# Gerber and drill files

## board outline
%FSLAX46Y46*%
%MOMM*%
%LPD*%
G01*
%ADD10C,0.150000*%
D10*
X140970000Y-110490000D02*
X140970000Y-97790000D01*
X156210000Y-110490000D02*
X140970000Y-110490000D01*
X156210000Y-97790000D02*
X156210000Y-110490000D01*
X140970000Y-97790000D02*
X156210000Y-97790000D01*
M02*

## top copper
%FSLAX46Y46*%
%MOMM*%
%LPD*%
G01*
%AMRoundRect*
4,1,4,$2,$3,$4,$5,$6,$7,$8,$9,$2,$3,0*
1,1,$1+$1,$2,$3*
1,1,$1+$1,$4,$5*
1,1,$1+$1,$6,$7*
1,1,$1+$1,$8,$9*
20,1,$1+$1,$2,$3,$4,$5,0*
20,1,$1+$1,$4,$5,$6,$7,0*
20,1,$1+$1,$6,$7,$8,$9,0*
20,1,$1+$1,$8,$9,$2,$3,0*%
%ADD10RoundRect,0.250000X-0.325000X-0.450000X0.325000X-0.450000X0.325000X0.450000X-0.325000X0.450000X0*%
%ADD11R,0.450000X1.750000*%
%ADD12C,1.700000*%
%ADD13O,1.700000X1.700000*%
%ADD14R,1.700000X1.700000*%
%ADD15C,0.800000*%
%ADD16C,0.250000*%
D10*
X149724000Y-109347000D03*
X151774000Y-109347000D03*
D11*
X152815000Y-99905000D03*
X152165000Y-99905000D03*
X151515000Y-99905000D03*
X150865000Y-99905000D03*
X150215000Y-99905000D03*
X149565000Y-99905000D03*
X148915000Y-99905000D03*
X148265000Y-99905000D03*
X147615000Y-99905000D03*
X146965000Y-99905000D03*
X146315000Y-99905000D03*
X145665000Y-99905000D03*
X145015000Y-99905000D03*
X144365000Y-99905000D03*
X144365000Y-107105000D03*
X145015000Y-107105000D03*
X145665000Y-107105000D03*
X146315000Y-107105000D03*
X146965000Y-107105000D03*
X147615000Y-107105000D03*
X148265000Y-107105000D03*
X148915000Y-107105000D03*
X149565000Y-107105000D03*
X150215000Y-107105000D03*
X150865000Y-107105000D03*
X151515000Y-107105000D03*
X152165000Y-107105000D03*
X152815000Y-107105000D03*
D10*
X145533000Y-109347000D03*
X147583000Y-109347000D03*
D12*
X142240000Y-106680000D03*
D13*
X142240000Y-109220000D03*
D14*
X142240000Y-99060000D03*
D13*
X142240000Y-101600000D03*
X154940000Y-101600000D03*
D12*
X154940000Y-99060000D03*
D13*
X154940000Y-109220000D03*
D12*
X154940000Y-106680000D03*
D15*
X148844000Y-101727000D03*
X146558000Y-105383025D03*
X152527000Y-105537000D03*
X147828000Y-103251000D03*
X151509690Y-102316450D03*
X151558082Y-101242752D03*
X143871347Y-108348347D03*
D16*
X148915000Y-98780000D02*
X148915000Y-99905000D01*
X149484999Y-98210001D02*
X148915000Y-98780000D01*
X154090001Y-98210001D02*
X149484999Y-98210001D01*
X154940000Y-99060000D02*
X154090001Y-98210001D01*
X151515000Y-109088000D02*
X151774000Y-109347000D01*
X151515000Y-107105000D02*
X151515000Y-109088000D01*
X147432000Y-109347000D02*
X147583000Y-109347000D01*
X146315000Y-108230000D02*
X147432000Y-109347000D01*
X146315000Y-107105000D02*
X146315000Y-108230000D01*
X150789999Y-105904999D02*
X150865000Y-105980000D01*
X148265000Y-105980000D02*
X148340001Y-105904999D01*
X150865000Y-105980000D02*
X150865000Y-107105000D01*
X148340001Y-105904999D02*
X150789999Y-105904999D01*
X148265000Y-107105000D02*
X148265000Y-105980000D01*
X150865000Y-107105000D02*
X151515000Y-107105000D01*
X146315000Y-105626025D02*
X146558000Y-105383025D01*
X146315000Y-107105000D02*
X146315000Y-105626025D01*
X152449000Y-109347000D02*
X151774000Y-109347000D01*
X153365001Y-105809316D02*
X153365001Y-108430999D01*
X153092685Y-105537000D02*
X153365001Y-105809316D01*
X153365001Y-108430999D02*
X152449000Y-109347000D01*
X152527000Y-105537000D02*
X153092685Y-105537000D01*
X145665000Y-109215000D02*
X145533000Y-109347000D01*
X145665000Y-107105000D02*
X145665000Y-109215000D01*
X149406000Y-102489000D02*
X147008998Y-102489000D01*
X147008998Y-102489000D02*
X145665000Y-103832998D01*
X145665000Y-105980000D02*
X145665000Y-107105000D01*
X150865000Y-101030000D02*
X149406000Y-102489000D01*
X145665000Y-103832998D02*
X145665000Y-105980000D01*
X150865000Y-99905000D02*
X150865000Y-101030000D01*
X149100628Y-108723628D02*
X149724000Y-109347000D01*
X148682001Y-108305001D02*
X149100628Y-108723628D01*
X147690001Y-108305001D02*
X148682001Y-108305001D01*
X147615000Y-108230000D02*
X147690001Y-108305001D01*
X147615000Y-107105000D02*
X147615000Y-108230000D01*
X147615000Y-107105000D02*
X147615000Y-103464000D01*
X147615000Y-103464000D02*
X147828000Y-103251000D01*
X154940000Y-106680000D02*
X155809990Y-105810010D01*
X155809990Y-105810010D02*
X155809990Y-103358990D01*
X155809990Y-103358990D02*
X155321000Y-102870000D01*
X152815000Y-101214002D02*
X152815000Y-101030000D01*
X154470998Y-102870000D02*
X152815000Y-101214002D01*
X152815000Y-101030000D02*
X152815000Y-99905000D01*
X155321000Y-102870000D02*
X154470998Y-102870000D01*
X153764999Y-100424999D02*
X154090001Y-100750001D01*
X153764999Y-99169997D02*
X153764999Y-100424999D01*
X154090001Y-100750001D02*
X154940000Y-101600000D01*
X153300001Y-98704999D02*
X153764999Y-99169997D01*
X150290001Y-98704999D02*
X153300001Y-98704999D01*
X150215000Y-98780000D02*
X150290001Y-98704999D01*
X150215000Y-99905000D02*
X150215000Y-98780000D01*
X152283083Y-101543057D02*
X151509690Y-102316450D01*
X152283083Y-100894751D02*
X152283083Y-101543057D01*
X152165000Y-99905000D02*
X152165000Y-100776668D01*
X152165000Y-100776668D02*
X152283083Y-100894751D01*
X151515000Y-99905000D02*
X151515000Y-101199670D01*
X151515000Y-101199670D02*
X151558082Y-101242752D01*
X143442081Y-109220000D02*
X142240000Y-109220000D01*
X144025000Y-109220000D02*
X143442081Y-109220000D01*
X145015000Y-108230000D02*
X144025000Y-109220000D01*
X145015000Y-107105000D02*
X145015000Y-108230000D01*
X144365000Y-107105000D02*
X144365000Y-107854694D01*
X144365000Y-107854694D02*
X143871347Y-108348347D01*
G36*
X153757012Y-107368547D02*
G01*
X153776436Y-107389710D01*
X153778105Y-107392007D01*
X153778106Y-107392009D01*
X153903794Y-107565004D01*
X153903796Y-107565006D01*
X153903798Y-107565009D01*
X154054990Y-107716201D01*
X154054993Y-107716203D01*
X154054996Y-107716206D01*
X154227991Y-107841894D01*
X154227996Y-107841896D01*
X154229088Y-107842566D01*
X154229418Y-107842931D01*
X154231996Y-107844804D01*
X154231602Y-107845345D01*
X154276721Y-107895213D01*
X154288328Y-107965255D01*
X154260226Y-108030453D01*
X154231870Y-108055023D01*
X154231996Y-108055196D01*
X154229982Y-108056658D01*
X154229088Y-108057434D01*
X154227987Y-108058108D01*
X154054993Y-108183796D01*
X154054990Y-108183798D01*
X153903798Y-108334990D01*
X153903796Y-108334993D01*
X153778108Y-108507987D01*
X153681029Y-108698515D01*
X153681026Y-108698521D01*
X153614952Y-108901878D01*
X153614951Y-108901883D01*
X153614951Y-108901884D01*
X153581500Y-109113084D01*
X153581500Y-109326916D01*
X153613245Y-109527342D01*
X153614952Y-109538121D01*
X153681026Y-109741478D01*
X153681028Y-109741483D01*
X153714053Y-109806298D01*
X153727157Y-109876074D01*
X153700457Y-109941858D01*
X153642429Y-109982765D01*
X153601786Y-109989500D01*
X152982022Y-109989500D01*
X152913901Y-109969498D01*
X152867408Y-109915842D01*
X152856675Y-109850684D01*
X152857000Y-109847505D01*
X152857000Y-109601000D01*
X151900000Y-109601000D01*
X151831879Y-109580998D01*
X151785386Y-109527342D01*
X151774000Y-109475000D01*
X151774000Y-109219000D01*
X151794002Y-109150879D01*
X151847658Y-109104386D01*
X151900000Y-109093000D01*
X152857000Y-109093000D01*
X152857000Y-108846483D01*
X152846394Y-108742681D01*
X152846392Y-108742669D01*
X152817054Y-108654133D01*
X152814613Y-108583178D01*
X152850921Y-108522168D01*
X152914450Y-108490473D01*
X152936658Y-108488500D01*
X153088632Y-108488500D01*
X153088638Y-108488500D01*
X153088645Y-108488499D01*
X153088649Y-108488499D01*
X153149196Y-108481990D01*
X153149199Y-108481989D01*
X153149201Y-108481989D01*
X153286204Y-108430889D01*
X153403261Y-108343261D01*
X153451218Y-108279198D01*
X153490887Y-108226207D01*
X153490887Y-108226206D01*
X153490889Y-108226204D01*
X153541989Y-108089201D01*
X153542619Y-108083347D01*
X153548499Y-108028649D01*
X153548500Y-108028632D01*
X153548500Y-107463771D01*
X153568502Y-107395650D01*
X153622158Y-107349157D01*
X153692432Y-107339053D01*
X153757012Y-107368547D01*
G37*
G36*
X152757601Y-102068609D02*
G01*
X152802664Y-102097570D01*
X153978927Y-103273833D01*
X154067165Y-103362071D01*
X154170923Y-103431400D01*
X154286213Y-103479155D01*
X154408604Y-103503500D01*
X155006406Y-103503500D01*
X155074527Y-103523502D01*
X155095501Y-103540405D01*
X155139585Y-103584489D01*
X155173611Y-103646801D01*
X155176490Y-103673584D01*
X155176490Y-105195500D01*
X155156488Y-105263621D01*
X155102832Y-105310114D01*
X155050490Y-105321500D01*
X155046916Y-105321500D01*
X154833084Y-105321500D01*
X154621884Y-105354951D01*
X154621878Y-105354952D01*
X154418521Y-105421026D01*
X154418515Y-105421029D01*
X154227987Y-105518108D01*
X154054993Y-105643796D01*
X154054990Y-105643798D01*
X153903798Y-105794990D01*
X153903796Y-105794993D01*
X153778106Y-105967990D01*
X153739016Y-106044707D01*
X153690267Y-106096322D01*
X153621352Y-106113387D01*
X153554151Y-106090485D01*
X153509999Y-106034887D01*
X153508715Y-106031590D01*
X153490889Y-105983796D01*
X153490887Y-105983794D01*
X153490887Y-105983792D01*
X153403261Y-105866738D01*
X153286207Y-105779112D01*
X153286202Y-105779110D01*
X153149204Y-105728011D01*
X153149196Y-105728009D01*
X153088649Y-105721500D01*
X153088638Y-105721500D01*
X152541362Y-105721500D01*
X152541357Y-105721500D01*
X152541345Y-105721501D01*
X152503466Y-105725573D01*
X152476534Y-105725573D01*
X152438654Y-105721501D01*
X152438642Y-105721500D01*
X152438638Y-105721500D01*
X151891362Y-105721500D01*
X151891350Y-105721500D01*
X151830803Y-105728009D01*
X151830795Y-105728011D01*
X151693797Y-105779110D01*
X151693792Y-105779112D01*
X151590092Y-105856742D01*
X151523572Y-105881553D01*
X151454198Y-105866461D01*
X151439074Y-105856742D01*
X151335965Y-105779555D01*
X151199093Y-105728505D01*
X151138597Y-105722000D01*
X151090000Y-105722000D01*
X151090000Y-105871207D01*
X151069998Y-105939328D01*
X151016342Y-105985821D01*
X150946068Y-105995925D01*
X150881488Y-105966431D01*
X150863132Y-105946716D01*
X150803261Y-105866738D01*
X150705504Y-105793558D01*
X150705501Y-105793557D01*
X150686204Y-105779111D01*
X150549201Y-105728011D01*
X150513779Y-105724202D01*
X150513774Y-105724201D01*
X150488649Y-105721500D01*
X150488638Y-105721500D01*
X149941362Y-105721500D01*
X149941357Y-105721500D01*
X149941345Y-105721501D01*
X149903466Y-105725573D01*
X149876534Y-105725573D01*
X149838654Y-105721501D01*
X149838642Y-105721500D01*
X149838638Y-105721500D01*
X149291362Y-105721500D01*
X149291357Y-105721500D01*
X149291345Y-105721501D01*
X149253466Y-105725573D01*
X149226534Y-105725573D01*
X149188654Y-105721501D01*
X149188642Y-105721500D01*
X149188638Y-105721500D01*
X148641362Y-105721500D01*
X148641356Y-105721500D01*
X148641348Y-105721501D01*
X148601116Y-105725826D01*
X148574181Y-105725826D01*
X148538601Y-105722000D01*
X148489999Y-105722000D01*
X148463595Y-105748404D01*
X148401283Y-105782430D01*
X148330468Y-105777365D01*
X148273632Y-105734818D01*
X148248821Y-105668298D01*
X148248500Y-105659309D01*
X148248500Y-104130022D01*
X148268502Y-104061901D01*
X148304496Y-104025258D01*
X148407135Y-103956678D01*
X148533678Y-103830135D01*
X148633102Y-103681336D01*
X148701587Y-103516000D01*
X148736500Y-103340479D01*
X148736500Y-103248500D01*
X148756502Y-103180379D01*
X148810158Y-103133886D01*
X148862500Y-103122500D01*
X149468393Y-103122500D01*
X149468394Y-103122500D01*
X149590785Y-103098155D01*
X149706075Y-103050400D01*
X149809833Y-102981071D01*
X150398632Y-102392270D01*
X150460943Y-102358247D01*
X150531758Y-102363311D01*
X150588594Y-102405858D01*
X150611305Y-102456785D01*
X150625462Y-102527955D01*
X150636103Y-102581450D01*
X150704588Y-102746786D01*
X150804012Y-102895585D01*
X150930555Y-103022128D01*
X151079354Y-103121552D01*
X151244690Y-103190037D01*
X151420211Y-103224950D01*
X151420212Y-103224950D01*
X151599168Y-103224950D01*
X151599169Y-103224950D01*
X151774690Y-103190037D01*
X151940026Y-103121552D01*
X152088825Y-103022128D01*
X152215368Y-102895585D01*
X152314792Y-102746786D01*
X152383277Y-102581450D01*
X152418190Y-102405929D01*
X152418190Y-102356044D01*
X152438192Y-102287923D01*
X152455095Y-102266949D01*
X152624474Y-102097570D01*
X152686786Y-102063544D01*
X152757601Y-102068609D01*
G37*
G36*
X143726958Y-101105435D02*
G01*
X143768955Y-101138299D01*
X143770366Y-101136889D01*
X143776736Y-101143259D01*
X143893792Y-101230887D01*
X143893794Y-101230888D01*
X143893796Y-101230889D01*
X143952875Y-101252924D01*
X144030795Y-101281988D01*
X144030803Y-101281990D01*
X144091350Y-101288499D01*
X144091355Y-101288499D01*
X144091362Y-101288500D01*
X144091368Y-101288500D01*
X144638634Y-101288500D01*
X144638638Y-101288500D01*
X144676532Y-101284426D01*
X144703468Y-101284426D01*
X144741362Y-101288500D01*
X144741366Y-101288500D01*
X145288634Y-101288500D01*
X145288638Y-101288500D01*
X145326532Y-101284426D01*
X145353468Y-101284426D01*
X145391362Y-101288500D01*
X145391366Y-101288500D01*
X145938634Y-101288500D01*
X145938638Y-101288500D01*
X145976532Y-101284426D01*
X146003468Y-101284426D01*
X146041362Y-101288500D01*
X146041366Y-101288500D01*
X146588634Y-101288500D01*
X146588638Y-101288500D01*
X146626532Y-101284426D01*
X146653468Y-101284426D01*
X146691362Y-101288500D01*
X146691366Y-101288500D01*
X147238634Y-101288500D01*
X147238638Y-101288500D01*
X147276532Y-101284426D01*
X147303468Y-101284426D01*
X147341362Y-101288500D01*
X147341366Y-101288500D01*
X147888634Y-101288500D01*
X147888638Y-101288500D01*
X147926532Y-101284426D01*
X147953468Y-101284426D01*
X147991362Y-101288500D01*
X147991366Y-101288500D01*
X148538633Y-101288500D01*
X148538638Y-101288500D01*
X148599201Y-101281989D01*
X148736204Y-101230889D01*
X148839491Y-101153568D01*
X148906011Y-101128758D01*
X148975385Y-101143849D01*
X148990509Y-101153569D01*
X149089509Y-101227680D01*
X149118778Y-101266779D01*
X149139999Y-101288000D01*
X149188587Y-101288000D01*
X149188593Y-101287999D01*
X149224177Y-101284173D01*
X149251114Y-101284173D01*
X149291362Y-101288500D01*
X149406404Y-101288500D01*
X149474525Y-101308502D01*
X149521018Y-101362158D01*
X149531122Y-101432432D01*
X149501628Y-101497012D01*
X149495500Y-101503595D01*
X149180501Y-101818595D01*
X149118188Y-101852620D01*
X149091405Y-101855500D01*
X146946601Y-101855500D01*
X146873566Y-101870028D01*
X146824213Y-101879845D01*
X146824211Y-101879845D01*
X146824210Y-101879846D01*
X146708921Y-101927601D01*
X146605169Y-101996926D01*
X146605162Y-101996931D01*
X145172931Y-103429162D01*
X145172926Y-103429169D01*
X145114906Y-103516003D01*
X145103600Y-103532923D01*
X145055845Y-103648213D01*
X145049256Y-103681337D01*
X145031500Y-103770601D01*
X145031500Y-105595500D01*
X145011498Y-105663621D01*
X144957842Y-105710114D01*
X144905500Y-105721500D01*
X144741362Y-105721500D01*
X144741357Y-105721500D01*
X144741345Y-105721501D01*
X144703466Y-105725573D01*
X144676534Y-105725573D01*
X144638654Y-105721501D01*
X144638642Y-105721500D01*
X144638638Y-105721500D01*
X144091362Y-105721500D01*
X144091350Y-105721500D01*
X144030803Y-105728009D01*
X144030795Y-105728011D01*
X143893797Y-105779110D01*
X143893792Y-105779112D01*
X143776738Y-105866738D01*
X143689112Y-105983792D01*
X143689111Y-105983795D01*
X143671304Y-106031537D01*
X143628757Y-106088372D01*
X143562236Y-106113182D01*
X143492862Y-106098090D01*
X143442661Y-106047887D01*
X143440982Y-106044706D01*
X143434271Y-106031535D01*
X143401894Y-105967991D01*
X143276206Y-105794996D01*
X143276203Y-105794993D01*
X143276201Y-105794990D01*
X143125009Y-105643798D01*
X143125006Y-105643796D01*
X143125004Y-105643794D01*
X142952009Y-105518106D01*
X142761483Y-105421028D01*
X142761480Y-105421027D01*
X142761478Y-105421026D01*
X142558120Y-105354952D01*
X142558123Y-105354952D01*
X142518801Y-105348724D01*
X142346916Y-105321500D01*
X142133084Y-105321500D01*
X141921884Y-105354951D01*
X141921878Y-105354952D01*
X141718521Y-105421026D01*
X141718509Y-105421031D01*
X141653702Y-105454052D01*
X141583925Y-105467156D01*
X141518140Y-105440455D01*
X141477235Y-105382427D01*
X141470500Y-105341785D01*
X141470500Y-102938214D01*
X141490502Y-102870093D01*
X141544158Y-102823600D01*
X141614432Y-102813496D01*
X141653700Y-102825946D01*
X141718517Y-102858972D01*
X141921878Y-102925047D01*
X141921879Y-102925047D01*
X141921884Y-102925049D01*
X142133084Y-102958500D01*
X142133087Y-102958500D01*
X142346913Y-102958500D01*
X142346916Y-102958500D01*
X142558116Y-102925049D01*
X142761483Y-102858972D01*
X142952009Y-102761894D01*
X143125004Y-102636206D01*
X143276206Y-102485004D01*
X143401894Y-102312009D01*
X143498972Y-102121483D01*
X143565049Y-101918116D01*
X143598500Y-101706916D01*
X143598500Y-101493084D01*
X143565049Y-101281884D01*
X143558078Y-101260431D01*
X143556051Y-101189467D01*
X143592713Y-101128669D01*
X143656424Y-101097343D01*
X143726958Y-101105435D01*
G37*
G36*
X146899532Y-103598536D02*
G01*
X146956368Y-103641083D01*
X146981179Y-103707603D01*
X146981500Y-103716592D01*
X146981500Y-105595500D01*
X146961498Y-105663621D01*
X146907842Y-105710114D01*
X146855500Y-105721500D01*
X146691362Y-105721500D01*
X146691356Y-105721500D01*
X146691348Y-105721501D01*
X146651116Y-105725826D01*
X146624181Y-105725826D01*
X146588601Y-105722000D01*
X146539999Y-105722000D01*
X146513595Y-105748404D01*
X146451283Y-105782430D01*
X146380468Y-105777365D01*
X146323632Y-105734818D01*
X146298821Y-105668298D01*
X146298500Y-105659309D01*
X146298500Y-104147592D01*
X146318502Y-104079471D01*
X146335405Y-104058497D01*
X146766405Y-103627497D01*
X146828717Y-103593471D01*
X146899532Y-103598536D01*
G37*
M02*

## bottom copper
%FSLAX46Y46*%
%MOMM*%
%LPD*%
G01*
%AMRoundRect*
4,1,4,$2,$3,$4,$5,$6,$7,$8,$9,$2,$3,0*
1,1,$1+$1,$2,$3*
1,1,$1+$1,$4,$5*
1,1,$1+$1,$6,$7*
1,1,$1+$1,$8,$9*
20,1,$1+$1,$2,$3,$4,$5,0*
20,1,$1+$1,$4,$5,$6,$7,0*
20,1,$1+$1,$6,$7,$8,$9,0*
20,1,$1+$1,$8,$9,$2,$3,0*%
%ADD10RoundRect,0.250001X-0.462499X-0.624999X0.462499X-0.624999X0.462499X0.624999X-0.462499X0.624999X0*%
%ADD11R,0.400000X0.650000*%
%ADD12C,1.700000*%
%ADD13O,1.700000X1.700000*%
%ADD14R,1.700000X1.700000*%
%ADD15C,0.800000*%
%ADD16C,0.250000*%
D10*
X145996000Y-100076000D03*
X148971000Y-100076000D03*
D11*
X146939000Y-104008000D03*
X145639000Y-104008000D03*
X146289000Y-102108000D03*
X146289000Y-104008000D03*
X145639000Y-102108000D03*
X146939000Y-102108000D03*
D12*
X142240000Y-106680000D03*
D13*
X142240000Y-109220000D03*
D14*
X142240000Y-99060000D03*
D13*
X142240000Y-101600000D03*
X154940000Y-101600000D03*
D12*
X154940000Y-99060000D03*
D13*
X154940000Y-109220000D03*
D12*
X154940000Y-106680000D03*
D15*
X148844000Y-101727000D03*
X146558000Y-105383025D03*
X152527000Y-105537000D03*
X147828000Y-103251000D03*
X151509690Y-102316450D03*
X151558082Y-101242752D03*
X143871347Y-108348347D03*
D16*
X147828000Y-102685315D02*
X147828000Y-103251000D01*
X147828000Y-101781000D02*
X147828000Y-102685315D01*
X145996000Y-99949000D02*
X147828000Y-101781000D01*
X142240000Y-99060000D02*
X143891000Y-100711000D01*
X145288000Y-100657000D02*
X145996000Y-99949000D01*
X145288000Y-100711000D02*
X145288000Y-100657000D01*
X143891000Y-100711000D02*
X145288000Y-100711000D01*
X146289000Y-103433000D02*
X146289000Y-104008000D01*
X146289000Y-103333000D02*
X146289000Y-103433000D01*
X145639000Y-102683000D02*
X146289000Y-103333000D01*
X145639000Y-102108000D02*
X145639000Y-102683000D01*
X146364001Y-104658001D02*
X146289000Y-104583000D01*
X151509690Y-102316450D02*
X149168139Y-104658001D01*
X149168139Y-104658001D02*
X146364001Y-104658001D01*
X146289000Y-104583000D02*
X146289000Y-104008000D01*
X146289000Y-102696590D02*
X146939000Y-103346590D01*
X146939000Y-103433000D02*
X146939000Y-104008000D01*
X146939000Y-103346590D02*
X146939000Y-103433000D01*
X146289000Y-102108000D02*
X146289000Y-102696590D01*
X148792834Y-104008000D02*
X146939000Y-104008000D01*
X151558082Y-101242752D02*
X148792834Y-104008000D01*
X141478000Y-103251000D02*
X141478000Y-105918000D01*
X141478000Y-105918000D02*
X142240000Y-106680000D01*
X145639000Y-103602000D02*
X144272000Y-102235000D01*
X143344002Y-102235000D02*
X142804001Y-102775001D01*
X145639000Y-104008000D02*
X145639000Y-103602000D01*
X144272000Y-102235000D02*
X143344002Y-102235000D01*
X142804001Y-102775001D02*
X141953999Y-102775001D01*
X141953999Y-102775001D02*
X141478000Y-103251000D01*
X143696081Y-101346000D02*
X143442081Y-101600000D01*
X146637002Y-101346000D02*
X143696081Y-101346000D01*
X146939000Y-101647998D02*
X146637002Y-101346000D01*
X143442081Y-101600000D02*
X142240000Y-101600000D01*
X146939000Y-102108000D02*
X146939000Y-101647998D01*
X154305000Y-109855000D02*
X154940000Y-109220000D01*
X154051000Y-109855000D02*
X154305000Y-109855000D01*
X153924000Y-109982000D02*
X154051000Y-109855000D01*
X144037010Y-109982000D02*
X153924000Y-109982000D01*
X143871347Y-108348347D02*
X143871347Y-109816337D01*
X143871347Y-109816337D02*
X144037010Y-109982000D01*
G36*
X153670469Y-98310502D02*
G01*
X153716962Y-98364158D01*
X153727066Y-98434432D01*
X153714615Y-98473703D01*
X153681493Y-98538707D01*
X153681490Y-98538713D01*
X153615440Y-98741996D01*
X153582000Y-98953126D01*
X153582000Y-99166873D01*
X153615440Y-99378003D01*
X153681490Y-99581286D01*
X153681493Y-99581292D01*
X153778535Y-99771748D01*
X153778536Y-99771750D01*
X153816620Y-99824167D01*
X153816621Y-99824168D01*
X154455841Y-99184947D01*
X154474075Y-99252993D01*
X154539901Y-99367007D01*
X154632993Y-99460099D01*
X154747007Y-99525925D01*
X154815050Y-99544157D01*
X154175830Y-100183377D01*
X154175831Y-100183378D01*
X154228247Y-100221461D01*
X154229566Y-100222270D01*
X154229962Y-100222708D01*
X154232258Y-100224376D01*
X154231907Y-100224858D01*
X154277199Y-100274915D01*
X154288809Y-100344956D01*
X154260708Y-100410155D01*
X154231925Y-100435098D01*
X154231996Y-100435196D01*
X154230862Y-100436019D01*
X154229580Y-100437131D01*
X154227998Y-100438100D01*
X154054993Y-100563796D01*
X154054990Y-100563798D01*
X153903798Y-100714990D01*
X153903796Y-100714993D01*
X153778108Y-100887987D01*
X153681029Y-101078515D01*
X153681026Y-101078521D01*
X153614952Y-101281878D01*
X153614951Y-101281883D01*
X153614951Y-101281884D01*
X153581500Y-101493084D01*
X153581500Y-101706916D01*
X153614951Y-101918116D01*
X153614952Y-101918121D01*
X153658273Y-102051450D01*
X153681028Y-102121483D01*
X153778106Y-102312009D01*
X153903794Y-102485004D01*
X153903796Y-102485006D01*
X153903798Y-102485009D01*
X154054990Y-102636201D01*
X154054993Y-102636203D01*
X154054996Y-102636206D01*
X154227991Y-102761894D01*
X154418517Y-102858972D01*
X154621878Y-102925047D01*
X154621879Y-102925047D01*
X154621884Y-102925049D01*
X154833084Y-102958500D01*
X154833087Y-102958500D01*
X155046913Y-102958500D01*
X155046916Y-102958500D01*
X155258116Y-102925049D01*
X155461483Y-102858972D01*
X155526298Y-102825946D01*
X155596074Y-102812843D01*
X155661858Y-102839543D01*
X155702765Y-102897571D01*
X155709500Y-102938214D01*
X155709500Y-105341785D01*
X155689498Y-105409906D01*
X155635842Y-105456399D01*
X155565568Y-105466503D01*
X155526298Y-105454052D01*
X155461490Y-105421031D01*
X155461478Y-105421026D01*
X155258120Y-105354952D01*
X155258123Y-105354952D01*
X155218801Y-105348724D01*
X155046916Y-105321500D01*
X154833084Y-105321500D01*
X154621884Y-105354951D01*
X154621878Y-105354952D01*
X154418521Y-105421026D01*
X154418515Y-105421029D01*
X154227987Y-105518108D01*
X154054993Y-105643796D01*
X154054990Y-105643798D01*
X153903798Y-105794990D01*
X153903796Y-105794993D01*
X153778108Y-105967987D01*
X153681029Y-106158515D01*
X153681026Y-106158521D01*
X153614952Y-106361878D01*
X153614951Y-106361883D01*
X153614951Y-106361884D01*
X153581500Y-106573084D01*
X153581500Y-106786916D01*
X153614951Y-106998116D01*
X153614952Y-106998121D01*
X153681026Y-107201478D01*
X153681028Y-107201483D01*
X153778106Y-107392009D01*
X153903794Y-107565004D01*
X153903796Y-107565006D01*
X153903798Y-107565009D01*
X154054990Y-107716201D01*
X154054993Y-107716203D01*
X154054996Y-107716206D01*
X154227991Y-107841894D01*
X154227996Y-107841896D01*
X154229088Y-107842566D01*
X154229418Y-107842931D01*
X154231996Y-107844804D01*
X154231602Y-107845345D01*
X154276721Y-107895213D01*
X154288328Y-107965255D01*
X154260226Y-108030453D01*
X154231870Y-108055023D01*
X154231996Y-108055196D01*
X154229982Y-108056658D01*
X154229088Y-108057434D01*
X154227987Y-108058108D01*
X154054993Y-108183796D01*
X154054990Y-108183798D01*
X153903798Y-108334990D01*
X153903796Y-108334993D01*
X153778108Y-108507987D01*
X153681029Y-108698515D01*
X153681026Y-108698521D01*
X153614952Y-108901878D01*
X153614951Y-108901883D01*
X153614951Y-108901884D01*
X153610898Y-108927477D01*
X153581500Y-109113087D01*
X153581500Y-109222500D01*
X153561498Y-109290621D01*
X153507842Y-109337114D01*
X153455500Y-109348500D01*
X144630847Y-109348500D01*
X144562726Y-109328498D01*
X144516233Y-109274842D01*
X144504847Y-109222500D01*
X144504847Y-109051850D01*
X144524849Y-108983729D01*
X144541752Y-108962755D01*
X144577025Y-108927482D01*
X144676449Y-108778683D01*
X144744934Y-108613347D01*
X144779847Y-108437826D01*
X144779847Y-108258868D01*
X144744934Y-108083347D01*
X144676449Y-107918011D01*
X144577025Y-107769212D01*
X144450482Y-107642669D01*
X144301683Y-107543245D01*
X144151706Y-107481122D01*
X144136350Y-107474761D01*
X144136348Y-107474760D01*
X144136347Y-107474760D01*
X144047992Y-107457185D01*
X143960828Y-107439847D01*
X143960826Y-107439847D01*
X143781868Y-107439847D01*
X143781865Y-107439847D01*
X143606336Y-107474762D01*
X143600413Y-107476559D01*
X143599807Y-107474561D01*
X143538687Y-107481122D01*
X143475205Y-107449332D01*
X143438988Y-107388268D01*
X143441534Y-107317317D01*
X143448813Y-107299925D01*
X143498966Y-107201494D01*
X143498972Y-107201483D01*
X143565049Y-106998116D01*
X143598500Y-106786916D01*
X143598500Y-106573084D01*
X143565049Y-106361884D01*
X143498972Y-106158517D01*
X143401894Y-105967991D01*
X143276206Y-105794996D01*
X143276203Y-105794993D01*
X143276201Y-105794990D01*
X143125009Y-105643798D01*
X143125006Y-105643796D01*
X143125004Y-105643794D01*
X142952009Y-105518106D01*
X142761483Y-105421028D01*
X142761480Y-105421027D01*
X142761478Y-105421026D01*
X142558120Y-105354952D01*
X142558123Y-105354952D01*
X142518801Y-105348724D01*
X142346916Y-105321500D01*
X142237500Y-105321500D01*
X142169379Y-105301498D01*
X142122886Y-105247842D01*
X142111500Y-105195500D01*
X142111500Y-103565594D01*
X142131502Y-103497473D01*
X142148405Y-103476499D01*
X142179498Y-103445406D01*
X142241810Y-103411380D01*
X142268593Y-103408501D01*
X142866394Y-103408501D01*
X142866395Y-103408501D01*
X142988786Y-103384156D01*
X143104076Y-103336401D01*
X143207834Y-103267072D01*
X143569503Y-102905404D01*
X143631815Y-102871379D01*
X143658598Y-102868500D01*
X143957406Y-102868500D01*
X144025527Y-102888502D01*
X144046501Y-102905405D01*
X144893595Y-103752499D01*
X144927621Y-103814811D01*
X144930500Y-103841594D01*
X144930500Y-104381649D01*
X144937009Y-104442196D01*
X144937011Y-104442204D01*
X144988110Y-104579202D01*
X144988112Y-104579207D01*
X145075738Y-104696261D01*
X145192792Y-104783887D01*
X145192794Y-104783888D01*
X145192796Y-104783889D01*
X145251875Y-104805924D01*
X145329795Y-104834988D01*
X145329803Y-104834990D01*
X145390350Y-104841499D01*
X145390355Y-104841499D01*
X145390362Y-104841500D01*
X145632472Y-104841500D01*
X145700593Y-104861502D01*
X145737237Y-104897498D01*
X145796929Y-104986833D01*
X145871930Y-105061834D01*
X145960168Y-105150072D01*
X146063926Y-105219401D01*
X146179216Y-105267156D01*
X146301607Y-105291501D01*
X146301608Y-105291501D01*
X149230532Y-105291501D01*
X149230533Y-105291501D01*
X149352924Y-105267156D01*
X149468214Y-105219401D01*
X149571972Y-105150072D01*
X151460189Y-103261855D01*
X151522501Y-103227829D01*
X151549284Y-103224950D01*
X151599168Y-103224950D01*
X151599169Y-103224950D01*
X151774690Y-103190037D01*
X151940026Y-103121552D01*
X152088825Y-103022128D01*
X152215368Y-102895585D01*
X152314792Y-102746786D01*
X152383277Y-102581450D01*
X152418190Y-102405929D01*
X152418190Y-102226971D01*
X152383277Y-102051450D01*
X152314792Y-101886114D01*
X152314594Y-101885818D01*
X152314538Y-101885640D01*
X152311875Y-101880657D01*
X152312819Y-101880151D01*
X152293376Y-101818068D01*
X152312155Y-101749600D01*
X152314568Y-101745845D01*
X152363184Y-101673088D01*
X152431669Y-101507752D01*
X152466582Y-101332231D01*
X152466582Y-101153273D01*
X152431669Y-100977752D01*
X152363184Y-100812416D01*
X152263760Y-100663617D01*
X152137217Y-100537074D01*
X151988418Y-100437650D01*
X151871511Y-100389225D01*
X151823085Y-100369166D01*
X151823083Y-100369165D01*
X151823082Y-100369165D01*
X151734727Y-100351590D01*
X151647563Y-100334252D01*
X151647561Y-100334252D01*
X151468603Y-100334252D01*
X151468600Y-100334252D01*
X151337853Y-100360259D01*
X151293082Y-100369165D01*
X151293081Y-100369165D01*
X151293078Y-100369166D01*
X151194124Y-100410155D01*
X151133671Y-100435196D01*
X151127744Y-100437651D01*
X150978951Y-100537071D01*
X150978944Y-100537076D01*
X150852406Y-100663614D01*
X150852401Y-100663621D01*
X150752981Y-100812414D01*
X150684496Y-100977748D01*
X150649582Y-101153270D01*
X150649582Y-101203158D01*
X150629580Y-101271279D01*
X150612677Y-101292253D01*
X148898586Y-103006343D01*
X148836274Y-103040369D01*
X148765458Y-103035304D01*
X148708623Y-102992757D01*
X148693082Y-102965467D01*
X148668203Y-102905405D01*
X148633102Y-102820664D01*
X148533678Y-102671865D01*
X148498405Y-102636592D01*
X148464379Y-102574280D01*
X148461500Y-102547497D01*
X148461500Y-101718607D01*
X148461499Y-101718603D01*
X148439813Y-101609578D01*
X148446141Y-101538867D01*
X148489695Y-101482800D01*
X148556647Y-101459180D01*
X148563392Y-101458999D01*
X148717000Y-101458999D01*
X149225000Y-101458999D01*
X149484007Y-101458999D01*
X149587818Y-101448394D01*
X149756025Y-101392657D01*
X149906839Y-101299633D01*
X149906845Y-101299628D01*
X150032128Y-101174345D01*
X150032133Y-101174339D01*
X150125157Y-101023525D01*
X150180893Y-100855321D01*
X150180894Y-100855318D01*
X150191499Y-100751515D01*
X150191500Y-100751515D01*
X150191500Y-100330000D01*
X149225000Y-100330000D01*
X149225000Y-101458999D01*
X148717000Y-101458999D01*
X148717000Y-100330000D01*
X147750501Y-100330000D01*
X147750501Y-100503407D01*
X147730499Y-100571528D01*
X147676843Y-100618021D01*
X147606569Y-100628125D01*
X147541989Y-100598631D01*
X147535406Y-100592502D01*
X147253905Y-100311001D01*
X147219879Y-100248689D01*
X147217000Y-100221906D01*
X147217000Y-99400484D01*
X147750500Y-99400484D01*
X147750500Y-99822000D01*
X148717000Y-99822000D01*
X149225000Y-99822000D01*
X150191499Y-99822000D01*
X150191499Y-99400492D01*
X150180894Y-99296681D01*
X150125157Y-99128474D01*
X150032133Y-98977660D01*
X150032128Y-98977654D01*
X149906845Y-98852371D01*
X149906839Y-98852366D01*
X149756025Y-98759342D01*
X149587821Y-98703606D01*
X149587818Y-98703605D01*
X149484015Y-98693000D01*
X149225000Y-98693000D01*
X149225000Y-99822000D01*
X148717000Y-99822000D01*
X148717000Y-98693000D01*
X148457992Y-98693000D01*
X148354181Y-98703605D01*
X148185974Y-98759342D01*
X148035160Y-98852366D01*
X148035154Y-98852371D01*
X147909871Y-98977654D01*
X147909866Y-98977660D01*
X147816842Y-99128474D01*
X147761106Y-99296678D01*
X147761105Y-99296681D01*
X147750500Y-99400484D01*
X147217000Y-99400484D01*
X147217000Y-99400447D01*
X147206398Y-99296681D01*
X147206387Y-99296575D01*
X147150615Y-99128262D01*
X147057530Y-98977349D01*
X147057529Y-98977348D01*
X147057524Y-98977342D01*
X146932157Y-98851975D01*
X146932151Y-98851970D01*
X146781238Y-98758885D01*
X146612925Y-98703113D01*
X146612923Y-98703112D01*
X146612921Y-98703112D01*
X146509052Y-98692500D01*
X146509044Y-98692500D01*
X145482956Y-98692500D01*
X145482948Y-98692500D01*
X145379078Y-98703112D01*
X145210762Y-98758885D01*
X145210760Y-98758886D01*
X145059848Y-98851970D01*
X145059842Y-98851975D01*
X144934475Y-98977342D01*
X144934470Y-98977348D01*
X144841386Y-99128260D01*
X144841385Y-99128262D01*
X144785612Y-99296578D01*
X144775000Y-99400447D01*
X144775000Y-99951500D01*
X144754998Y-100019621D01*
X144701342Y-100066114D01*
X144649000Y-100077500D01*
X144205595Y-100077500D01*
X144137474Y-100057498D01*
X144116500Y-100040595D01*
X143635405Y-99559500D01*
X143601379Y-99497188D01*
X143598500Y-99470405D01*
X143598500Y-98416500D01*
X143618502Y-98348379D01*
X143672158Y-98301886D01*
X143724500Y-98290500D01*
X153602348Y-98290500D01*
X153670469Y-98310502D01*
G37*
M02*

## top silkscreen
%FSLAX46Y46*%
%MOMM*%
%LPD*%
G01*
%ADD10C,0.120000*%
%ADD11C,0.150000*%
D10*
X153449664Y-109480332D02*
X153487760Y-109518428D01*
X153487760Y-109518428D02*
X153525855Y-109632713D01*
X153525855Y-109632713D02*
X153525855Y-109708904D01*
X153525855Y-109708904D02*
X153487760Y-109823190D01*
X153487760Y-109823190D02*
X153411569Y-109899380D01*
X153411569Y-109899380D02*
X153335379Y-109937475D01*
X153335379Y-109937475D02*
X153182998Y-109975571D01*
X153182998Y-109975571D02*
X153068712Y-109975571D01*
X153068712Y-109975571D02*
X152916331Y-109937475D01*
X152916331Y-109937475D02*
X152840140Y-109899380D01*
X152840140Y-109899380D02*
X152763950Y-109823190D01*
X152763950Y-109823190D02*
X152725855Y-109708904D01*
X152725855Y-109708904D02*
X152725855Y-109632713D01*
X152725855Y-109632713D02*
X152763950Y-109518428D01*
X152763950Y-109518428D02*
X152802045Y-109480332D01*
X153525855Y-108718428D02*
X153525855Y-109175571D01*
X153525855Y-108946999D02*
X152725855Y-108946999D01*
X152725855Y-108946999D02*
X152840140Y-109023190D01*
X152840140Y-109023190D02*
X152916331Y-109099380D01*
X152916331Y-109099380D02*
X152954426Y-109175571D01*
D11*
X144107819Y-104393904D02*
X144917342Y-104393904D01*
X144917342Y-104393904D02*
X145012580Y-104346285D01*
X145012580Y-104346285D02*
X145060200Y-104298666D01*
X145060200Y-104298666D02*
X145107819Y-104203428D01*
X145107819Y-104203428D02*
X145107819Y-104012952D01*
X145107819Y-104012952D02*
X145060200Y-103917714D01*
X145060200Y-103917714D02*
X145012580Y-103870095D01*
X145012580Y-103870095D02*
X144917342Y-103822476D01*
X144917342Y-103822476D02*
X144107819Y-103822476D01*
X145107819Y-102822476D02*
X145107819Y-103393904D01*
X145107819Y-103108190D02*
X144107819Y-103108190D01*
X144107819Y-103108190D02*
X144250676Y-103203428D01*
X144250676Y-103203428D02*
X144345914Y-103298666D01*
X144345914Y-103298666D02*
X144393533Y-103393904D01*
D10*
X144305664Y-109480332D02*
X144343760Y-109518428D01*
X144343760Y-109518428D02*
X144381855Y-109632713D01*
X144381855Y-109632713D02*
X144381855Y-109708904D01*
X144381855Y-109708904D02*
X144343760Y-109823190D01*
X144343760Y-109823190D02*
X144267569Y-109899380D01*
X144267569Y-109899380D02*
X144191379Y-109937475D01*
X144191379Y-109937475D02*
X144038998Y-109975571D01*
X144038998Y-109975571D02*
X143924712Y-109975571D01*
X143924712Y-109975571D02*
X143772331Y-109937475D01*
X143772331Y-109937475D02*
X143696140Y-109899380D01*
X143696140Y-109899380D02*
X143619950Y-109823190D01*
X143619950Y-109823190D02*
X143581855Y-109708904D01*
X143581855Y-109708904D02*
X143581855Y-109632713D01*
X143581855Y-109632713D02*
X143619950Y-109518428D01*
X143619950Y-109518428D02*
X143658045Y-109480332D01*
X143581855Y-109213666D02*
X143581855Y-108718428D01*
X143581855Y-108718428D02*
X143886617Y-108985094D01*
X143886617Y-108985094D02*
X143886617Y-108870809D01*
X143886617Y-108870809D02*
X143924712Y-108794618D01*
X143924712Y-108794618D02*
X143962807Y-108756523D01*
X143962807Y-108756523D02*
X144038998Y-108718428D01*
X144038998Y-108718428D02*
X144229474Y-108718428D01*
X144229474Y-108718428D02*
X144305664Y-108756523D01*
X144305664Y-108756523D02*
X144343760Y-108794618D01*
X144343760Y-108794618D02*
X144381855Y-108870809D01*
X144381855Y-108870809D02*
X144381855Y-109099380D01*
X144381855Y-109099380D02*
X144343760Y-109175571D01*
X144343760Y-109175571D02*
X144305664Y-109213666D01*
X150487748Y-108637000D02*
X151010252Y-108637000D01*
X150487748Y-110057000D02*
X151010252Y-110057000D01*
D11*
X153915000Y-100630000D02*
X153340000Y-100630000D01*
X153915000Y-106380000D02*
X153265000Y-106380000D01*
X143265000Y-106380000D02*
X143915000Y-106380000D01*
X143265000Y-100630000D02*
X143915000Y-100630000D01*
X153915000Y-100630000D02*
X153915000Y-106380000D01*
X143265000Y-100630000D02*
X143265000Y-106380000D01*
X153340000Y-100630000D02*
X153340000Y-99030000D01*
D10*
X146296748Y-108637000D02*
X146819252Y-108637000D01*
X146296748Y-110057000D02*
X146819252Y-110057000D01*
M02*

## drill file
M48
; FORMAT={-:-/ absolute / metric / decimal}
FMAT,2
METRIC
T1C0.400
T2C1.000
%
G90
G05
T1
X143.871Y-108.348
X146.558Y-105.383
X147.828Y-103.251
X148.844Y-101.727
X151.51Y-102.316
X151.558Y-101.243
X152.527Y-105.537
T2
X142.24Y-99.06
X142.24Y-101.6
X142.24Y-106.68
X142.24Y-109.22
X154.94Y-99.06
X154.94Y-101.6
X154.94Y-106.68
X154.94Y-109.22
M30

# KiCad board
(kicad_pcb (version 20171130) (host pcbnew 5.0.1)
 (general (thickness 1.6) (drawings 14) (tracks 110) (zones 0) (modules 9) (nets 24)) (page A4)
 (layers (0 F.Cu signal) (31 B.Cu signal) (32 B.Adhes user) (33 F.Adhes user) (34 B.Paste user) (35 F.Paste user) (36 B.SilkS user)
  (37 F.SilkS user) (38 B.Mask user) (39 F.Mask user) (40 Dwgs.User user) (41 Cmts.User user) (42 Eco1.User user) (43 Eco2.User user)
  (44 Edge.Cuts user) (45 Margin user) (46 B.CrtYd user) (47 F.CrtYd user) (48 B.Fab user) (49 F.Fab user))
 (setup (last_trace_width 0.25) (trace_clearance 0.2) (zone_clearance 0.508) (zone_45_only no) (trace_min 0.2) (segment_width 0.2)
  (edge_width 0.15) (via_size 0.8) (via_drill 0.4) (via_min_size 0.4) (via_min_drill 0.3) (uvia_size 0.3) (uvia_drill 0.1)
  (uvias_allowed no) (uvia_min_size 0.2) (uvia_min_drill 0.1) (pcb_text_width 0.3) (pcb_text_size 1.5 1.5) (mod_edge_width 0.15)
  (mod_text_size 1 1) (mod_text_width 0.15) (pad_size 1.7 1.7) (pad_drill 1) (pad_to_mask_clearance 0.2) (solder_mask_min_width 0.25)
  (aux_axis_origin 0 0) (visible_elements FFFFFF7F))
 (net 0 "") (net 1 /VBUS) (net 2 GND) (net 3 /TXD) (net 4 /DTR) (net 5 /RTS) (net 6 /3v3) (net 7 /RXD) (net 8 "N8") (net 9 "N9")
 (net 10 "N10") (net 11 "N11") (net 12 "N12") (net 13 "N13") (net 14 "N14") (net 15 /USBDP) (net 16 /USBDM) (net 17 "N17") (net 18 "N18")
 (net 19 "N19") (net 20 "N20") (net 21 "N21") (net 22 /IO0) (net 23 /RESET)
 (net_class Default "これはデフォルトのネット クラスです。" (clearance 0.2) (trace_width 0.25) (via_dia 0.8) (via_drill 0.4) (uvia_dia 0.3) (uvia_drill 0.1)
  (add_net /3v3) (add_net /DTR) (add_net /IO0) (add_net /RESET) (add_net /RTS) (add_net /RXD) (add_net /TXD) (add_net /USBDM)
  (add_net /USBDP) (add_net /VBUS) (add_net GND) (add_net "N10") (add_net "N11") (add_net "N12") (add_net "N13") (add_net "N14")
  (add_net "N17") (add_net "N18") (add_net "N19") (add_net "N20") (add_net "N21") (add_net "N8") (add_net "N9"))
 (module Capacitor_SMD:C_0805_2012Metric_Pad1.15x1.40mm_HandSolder (layer F.Cu) (at 150.749 109.347)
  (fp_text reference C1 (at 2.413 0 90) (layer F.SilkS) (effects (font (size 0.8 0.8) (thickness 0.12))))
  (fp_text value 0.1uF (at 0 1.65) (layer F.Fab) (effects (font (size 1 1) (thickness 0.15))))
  (fp_line (start -0.261252 -0.71) (end 0.261252 -0.71) (layer F.SilkS) (width 0.12))
  (fp_line (start -0.261252 0.71) (end 0.261252 0.71) (layer F.SilkS) (width 0.12))
  (pad 1 smd roundrect (at -1.025 0) (size 1.15 1.4) (layers F.Cu F.Paste F.Mask) (roundrect_rratio 0.217391) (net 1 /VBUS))
  (pad 2 smd roundrect (at 1.025 0) (size 1.15 1.4) (layers F.Cu F.Paste F.Mask) (roundrect_rratio 0.217391) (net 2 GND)))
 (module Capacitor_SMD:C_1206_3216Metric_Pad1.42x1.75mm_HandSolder (layer B.Cu) (at 147.4835 100.076)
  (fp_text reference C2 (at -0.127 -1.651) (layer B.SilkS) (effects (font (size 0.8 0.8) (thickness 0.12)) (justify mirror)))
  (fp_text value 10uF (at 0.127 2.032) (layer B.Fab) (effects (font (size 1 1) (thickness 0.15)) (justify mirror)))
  (pad 1 smd roundrect (at -1.4875 0) (size 1.425 1.75) (layers B.Cu B.Paste B.Mask) (roundrect_rratio 0.175439) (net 1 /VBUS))
  (pad 2 smd roundrect (at 1.4875 0) (size 1.425 1.75) (layers B.Cu B.Paste B.Mask) (roundrect_rratio 0.175439) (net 2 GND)))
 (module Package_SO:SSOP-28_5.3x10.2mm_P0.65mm (layer F.Cu) (at 148.59 103.505 270)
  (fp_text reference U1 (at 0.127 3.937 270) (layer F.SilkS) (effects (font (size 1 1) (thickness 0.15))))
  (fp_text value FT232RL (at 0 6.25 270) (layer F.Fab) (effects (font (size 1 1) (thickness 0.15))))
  (fp_line (start -2.875 -5.325) (end -2.875 -4.75) (layer F.SilkS) (width 0.15))
  (fp_line (start 2.875 -5.325) (end 2.875 -4.675) (layer F.SilkS) (width 0.15))
  (fp_line (start 2.875 5.325) (end 2.875 4.675) (layer F.SilkS) (width 0.15))
  (fp_line (start -2.875 5.325) (end -2.875 4.675) (layer F.SilkS) (width 0.15))
  (fp_line (start -2.875 -5.325) (end 2.875 -5.325) (layer F.SilkS) (width 0.15))
  (fp_line (start -2.875 5.325) (end 2.875 5.325) (layer F.SilkS) (width 0.15))
  (fp_line (start -2.875 -4.75) (end -4.475 -4.75) (layer F.SilkS) (width 0.15))
  (pad 1 smd rect (at -3.6 -4.225 270) (size 1.75 0.45) (layers F.Cu F.Paste F.Mask) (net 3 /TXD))
  (pad 2 smd rect (at -3.6 -3.575 270) (size 1.75 0.45) (layers F.Cu F.Paste F.Mask) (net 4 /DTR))
  (pad 3 smd rect (at -3.6 -2.925 270) (size 1.75 0.45) (layers F.Cu F.Paste F.Mask) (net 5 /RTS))
  (pad 4 smd rect (at -3.6 -2.275 270) (size 1.75 0.45) (layers F.Cu F.Paste F.Mask) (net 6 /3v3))
  (pad 5 smd rect (at -3.6 -1.625 270) (size 1.75 0.45) (layers F.Cu F.Paste F.Mask) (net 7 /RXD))
  (pad 6 smd rect (at -3.6 -0.975 270) (size 1.75 0.45) (layers F.Cu F.Paste F.Mask) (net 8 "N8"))
  (pad 7 smd rect (at -3.6 -0.325 270) (size 1.75 0.45) (layers F.Cu F.Paste F.Mask) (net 2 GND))
  (pad 8 smd rect (at -3.6 0.325 270) (size 1.75 0.45) (layers F.Cu F.Paste F.Mask))
  (pad 9 smd rect (at -3.6 0.975 270) (size 1.75 0.45) (layers F.Cu F.Paste F.Mask) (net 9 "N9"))
  (pad 10 smd rect (at -3.6 1.625 270) (size 1.75 0.45) (layers F.Cu F.Paste F.Mask) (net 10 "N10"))
  (pad 11 smd rect (at -3.6 2.275 270) (size 1.75 0.45) (layers F.Cu F.Paste F.Mask) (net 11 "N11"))
  (pad 12 smd rect (at -3.6 2.925 270) (size 1.75 0.45) (layers F.Cu F.Paste F.Mask) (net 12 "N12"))
  (pad 13 smd rect (at -3.6 3.575 270) (size 1.75 0.45) (layers F.Cu F.Paste F.Mask) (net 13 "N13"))
  (pad 14 smd rect (at -3.6 4.225 270) (size 1.75 0.45) (layers F.Cu F.Paste F.Mask) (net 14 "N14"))
  (pad 15 smd rect (at 3.6 4.225 270) (size 1.75 0.45) (layers F.Cu F.Paste F.Mask) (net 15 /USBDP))
  (pad 16 smd rect (at 3.6 3.575 270) (size 1.75 0.45) (layers F.Cu F.Paste F.Mask) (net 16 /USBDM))
  (pad 17 smd rect (at 3.6 2.925 270) (size 1.75 0.45) (layers F.Cu F.Paste F.Mask) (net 6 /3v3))
  (pad 18 smd rect (at 3.6 2.275 270) (size 1.75 0.45) (layers F.Cu F.Paste F.Mask) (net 2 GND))
  (pad 19 smd rect (at 3.6 1.625 270) (size 1.75 0.45) (layers F.Cu F.Paste F.Mask) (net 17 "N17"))
  (pad 20 smd rect (at 3.6 0.975 270) (size 1.75 0.45) (layers F.Cu F.Paste F.Mask) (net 1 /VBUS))
  (pad 21 smd rect (at 3.6 0.325 270) (size 1.75 0.45) (layers F.Cu F.Paste F.Mask) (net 2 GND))
  (pad 22 smd rect (at 3.6 -0.325 270) (size 1.75 0.45) (layers F.Cu F.Paste F.Mask) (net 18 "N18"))
  (pad 23 smd rect (at 3.6 -0.975 270) (size 1.75 0.45) (layers F.Cu F.Paste F.Mask) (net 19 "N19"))
  (pad 24 smd rect (at 3.6 -1.625 270) (size 1.75 0.45) (layers F.Cu F.Paste F.Mask))
  (pad 25 smd rect (at 3.6 -2.275 270) (size 1.75 0.45) (layers F.Cu F.Paste F.Mask) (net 2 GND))
  (pad 26 smd rect (at 3.6 -2.925 270) (size 1.75 0.45) (layers F.Cu F.Paste F.Mask) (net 2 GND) (zone_connect 2))
  (pad 27 smd rect (at 3.6 -3.575 270) (size 1.75 0.45) (layers F.Cu F.Paste F.Mask) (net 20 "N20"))
  (pad 28 smd rect (at 3.6 -4.225 270) (size 1.75 0.45) (layers F.Cu F.Paste F.Mask) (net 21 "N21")))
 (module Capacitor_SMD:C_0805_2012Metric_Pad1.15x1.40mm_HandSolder (layer F.Cu) (at 146.558 109.347)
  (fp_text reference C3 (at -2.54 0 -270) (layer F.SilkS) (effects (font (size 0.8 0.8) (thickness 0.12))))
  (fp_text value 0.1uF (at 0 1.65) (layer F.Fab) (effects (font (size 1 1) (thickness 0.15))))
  (fp_line (start -0.261252 -0.71) (end 0.261252 -0.71) (layer F.SilkS) (width 0.12))
  (fp_line (start -0.261252 0.71) (end 0.261252 0.71) (layer F.SilkS) (width 0.12))
  (pad 1 smd roundrect (at -1.025 0) (size 1.15 1.4) (layers F.Cu F.Paste F.Mask) (roundrect_rratio 0.217391) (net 6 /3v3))
  (pad 2 smd roundrect (at 1.025 0) (size 1.15 1.4) (layers F.Cu F.Paste F.Mask) (roundrect_rratio 0.217391) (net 2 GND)))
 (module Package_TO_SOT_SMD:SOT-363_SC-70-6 (layer B.Cu) (at 146.289 103.058 90)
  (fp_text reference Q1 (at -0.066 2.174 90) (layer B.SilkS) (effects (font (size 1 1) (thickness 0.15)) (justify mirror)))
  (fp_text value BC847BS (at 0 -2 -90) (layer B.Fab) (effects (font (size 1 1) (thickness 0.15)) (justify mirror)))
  (pad 1 smd rect (at -0.95 0.65 90) (size 0.65 0.4) (layers B.Cu B.Paste B.Mask) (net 5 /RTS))
  (pad 3 smd rect (at -0.95 -0.65 90) (size 0.65 0.4) (layers B.Cu B.Paste B.Mask) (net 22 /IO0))
  (pad 5 smd rect (at 0.95 0 90) (size 0.65 0.4) (layers B.Cu B.Paste B.Mask) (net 5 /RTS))
  (pad 2 smd rect (at -0.95 0 90) (size 0.65 0.4) (layers B.Cu B.Paste B.Mask) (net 4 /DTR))
  (pad 4 smd rect (at 0.95 -0.65 90) (size 0.65 0.4) (layers B.Cu B.Paste B.Mask) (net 4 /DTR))
  (pad 6 smd rect (at 0.95 0.65 90) (size 0.65 0.4) (layers B.Cu B.Paste B.Mask) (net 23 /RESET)))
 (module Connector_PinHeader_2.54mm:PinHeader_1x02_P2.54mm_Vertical (layer B.Cu) (at 142.24 106.68 180)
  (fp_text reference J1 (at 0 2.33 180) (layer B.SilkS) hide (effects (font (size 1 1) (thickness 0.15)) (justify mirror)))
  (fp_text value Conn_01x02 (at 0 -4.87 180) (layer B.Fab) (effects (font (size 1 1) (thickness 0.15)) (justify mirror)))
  (pad 1 thru_hole circle (at 0 0 180) (size 1.7 1.7) (drill 1) (layers *.Cu *.Mask) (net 22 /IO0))
  (pad 2 thru_hole oval (at 0 -2.54 180) (size 1.7 1.7) (drill 1) (layers *.Cu *.Mask) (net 16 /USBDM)))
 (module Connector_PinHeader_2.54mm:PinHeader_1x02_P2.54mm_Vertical (layer B.Cu) (at 142.24 99.06 180)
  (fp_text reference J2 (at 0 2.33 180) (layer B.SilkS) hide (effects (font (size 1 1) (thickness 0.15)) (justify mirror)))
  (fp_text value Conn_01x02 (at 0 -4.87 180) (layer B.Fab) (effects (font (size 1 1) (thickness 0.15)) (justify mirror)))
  (pad 1 thru_hole rect (at 0 0 180) (size 1.7 1.7) (drill 1) (layers *.Cu *.Mask) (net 1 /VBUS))
  (pad 2 thru_hole oval (at 0 -2.54 180) (size 1.7 1.7) (drill 1) (layers *.Cu *.Mask) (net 23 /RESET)))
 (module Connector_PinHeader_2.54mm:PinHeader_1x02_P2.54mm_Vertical (layer B.Cu) (at 154.94 99.06 180)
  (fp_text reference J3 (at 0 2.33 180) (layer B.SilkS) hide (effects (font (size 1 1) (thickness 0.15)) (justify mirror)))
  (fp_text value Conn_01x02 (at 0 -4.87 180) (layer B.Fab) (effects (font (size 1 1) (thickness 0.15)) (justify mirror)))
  (pad 2 thru_hole oval (at 0 -2.54 180) (size 1.7 1.7) (drill 1) (layers *.Cu *.Mask) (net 7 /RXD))
  (pad 1 thru_hole circle (at 0 0 180) (size 1.7 1.7) (drill 1) (layers *.Cu *.Mask) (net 2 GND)))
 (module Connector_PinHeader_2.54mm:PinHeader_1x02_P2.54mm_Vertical (layer B.Cu) (at 154.94 106.68 180)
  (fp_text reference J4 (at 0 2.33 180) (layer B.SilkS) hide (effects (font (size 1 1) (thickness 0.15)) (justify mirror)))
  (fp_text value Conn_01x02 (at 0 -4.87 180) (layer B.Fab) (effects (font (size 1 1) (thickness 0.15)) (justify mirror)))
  (pad 2 thru_hole oval (at 0 -2.54 180) (size 1.7 1.7) (drill 1) (layers *.Cu *.Mask) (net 15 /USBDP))
  (pad 1 thru_hole circle (at 0 0 180) (size 1.7 1.7) (drill 1) (layers *.Cu *.Mask) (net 3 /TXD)))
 (gr_line (start 140.97 110.49) (end 140.97 97.79) (layer Edge.Cuts) (width 0.15))
 (gr_line (start 156.21 110.49) (end 140.97 110.49) (layer Edge.Cuts) (width 0.15))
 (gr_line (start 156.21 97.79) (end 156.21 110.49) (layer Edge.Cuts) (width 0.15))
 (gr_line (start 140.97 97.79) (end 156.21 97.79) (layer Edge.Cuts) (width 0.15))
 (segment (start 148.915 98.78) (end 148.915 99.905) (width 0.25) (layer F.Cu) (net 2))
 (segment (start 149.484999 98.210001) (end 148.915 98.78) (width 0.25) (layer F.Cu) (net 2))
 (segment (start 154.090001 98.210001) (end 149.484999 98.210001) (width 0.25) (layer F.Cu) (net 2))
 (segment (start 154.94 99.06) (end 154.090001 98.210001) (width 0.25) (layer F.Cu) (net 2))
 (segment (start 151.515 109.088) (end 151.774 109.347) (width 0.25) (layer F.Cu) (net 2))
 (segment (start 151.515 107.105) (end 151.515 109.088) (width 0.25) (layer F.Cu) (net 2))
 (segment (start 147.432 109.347) (end 147.583 109.347) (width 0.25) (layer F.Cu) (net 2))
 (segment (start 146.315 108.23) (end 147.432 109.347) (width 0.25) (layer F.Cu) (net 2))
 (segment (start 146.315 107.105) (end 146.315 108.23) (width 0.25) (layer F.Cu) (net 2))
 (segment (start 150.789999 105.904999) (end 150.865 105.98) (width 0.25) (layer F.Cu) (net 2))
 (segment (start 148.265 105.98) (end 148.340001 105.904999) (width 0.25) (layer F.Cu) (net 2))
 (segment (start 150.865 105.98) (end 150.865 107.105) (width 0.25) (layer F.Cu) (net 2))
 (segment (start 148.340001 105.904999) (end 150.789999 105.904999) (width 0.25) (layer F.Cu) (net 2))
 (segment (start 148.265 107.105) (end 148.265 105.98) (width 0.25) (layer F.Cu) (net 2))
 (segment (start 150.865 107.105) (end 151.515 107.105) (width 0.25) (layer F.Cu) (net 2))
 (via (at 148.844 101.727) (size 0.8) (drill 0.4) (layers F.Cu B.Cu) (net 2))
 (segment (start 146.315 105.626025) (end 146.558 105.383025) (width 0.25) (layer F.Cu) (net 2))
 (via (at 146.558 105.383025) (size 0.8) (drill 0.4) (layers F.Cu B.Cu) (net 2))
 (segment (start 146.315 107.105) (end 146.315 105.626025) (width 0.25) (layer F.Cu) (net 2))
 (via (at 152.527 105.537) (size 0.8) (drill 0.4) (layers F.Cu B.Cu) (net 2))
 (segment (start 152.449 109.347) (end 151.774 109.347) (width 0.25) (layer F.Cu) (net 2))
 (segment (start 153.365001 105.809316) (end 153.365001 108.430999) (width 0.25) (layer F.Cu) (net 2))
 (segment (start 153.092685 105.537) (end 153.365001 105.809316) (width 0.25) (layer F.Cu) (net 2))
 (segment (start 153.365001 108.430999) (end 152.449 109.347) (width 0.25) (layer F.Cu) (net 2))
 (segment (start 152.527 105.537) (end 153.092685 105.537) (width 0.25) (layer F.Cu) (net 2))
 (segment (start 145.665 109.215) (end 145.533 109.347) (width 0.25) (layer F.Cu) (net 6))
 (segment (start 145.665 107.105) (end 145.665 109.215) (width 0.25) (layer F.Cu) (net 6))
 (segment (start 149.406 102.489) (end 147.008998 102.489) (width 0.25) (layer F.Cu) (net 6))
 (segment (start 147.008998 102.489) (end 145.665 103.832998) (width 0.25) (layer F.Cu) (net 6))
 (segment (start 145.665 105.98) (end 145.665 107.105) (width 0.25) (layer F.Cu) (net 6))
 (segment (start 150.865 101.03) (end 149.406 102.489) (width 0.25) (layer F.Cu) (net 6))
 (segment (start 145.665 103.832998) (end 145.665 105.98) (width 0.25) (layer F.Cu) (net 6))
 (segment (start 150.865 99.905) (end 150.865 101.03) (width 0.25) (layer F.Cu) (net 6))
 (segment (start 149.100628 108.723628) (end 149.724 109.347) (width 0.25) (layer F.Cu) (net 1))
 (segment (start 148.682001 108.305001) (end 149.100628 108.723628) (width 0.25) (layer F.Cu) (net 1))
 (segment (start 147.690001 108.305001) (end 148.682001 108.305001) (width 0.25) (layer F.Cu) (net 1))
 (segment (start 147.615 108.23) (end 147.690001 108.305001) (width 0.25) (layer F.Cu) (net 1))
 (segment (start 147.615 107.105) (end 147.615 108.23) (width 0.25) (layer F.Cu) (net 1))
 (segment (start 147.615 107.105) (end 147.615 103.464) (width 0.25) (layer F.Cu) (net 1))
 (segment (start 147.615 103.464) (end 147.828 103.251) (width 0.25) (layer F.Cu) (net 1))
 (via (at 147.828 103.251) (size 0.8) (drill 0.4) (layers F.Cu B.Cu) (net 1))
 (segment (start 147.828 102.685315) (end 147.828 103.251) (width 0.25) (layer B.Cu) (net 1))
 (segment (start 147.828 101.781) (end 147.828 102.685315) (width 0.25) (layer B.Cu) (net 1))
 (segment (start 145.996 99.949) (end 147.828 101.781) (width 0.25) (layer B.Cu) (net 1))
 (segment (start 142.24 99.06) (end 143.891 100.711) (width 0.25) (layer B.Cu) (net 1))
 (segment (start 145.288 100.657) (end 145.996 99.949) (width 0.25) (layer B.Cu) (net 1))
 (segment (start 145.288 100.711) (end 145.288 100.657) (width 0.25) (layer B.Cu) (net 1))
 (segment (start 143.891 100.711) (end 145.288 100.711) (width 0.25) (layer B.Cu) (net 1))
 (segment (start 154.94 106.68) (end 155.80999 105.81001) (width 0.25) (layer F.Cu) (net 3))
 (segment (start 155.80999 105.81001) (end 155.80999 103.35899) (width 0.25) (layer F.Cu) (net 3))
 (segment (start 155.80999 103.35899) (end 155.321 102.87) (width 0.25) (layer F.Cu) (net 3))
 (segment (start 152.815 101.214002) (end 152.815 101.03) (width 0.25) (layer F.Cu) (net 3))
 (segment (start 154.470998 102.87) (end 152.815 101.214002) (width 0.25) (layer F.Cu) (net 3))
 (segment (start 152.815 101.03) (end 152.815 99.905) (width 0.25) (layer F.Cu) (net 3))
 (segment (start 155.321 102.87) (end 154.470998 102.87) (width 0.25) (layer F.Cu) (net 3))
 (segment (start 153.764999 100.424999) (end 154.090001 100.750001) (width 0.25) (layer F.Cu) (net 7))
 (segment (start 153.764999 99.169997) (end 153.764999 100.424999) (width 0.25) (layer F.Cu) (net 7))
 (segment (start 154.090001 100.750001) (end 154.94 101.6) (width 0.25) (layer F.Cu) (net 7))
 (segment (start 153.300001 98.704999) (end 153.764999 99.169997) (width 0.25) (layer F.Cu) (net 7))
 (segment (start 150.290001 98.704999) (end 153.300001 98.704999) (width 0.25) (layer F.Cu) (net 7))
 (segment (start 150.215 98.78) (end 150.290001 98.704999) (width 0.25) (layer F.Cu) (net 7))
 (segment (start 150.215 99.905) (end 150.215 98.78) (width 0.25) (layer F.Cu) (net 7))
 (segment (start 146.289 103.433) (end 146.289 104.008) (width 0.25) (layer B.Cu) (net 4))
 (segment (start 146.289 103.333) (end 146.289 103.433) (width 0.25) (layer B.Cu) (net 4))
 (segment (start 145.639 102.683) (end 146.289 103.333) (width 0.25) (layer B.Cu) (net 4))
 (segment (start 145.639 102.108) (end 145.639 102.683) (width 0.25) (layer B.Cu) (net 4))
 (via (at 151.50969 102.31645) (size 0.8) (drill 0.4) (layers F.Cu B.Cu) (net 4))
 (segment (start 152.283083 101.543057) (end 151.50969 102.31645) (width 0.25) (layer F.Cu) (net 4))
 (segment (start 152.283083 100.894751) (end 152.283083 101.543057) (width 0.25) (layer F.Cu) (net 4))
 (segment (start 152.165 99.905) (end 152.165 100.776668) (width 0.25) (layer F.Cu) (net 4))
 (segment (start 152.165 100.776668) (end 152.283083 100.894751) (width 0.25) (layer F.Cu) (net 4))
 (segment (start 146.364001 104.658001) (end 146.289 104.583) (width 0.25) (layer B.Cu) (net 4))
 (segment (start 151.50969 102.31645) (end 149.168139 104.658001) (width 0.25) (layer B.Cu) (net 4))
 (segment (start 149.168139 104.658001) (end 146.364001 104.658001) (width 0.25) (layer B.Cu) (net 4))
 (segment (start 146.289 104.583) (end 146.289 104.008) (width 0.25) (layer B.Cu) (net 4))
 (segment (start 146.289 102.69659) (end 146.939 103.34659) (width 0.25) (layer B.Cu) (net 5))
 (segment (start 146.939 103.433) (end 146.939 104.008) (width 0.25) (layer B.Cu) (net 5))
 (segment (start 146.939 103.34659) (end 146.939 103.433) (width 0.25) (layer B.Cu) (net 5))
 (segment (start 146.289 102.108) (end 146.289 102.69659) (width 0.25) (layer B.Cu) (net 5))
 (segment (start 151.515 99.905) (end 151.515 101.19967) (width 0.25) (layer F.Cu) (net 5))
 (via (at 151.558082 101.242752) (size 0.8) (drill 0.4) (layers F.Cu B.Cu) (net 5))
 (segment (start 151.515 101.19967) (end 151.558082 101.242752) (width 0.25) (layer F.Cu) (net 5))
 (segment (start 148.792834 104.008) (end 146.939 104.008) (width 0.25) (layer B.Cu) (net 5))
 (segment (start 151.558082 101.242752) (end 148.792834 104.008) (width 0.25) (layer B.Cu) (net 5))
 (segment (start 141.478 103.251) (end 141.478 105.918) (width 0.25) (layer B.Cu) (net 22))
 (segment (start 141.478 105.918) (end 142.24 106.68) (width 0.25) (layer B.Cu) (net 22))
 (segment (start 145.639 103.602) (end 144.272 102.235) (width 0.25) (layer B.Cu) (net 22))
 (segment (start 143.344002 102.235) (end 142.804001 102.775001) (width 0.25) (layer B.Cu) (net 22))
 (segment (start 145.639 104.008) (end 145.639 103.602) (width 0.25) (layer B.Cu) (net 22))
 (segment (start 144.272 102.235) (end 143.344002 102.235) (width 0.25) (layer B.Cu) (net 22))
 (segment (start 142.804001 102.775001) (end 141.953999 102.775001) (width 0.25) (layer B.Cu) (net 22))
 (segment (start 141.953999 102.775001) (end 141.478 103.251) (width 0.25) (layer B.Cu) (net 22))
 (segment (start 143.696081 101.346) (end 143.442081 101.6) (width 0.25) (layer B.Cu) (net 23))
 (segment (start 146.637002 101.346) (end 143.696081 101.346) (width 0.25) (layer B.Cu) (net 23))
 (segment (start 146.939 101.647998) (end 146.637002 101.346) (width 0.25) (layer B.Cu) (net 23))
 (segment (start 143.442081 101.6) (end 142.24 101.6) (width 0.25) (layer B.Cu) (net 23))
 (segment (start 146.939 102.108) (end 146.939 101.647998) (width 0.25) (layer B.Cu) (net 23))
 (segment (start 143.442081 109.22) (end 142.24 109.22) (width 0.25) (layer F.Cu) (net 16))
 (segment (start 144.025 109.22) (end 143.442081 109.22) (width 0.25) (layer F.Cu) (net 16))
 (segment (start 145.015 108.23) (end 144.025 109.22) (width 0.25) (layer F.Cu) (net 16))
 (segment (start 145.015 107.105) (end 145.015 108.23) (width 0.25) (layer F.Cu) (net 16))
 (via (at 143.871347 108.348347) (size 0.8) (drill 0.4) (layers F.Cu B.Cu) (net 15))
 (segment (start 144.365 107.105) (end 144.365 107.854694) (width 0.25) (layer F.Cu) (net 15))
 (segment (start 144.365 107.854694) (end 143.871347 108.348347) (width 0.25) (layer F.Cu) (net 15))
 (segment (start 154.305 109.855) (end 154.94 109.22) (width 0.25) (layer B.Cu) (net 15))
 (segment (start 154.051 109.855) (end 154.305 109.855) (width 0.25) (layer B.Cu) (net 15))
 (segment (start 153.924 109.982) (end 154.051 109.855) (width 0.25) (layer B.Cu) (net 15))
 (segment (start 144.03701 109.982) (end 153.924 109.982) (width 0.25) (layer B.Cu) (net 15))
 (segment (start 143.871347 108.348347) (end 143.871347 109.816337) (width 0.25) (layer B.Cu) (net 15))
 (segment (start 143.871347 109.816337) (end 144.03701 109.982) (width 0.25) (layer B.Cu) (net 15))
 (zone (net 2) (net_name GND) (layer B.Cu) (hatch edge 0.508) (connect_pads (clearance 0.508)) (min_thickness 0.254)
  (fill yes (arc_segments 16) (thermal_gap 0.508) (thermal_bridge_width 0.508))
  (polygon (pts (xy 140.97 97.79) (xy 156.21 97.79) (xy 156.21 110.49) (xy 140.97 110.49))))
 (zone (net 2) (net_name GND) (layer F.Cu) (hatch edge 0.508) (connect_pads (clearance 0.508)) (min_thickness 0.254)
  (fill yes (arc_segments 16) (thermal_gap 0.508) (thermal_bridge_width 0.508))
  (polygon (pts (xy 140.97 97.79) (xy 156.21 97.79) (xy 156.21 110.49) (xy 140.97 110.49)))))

